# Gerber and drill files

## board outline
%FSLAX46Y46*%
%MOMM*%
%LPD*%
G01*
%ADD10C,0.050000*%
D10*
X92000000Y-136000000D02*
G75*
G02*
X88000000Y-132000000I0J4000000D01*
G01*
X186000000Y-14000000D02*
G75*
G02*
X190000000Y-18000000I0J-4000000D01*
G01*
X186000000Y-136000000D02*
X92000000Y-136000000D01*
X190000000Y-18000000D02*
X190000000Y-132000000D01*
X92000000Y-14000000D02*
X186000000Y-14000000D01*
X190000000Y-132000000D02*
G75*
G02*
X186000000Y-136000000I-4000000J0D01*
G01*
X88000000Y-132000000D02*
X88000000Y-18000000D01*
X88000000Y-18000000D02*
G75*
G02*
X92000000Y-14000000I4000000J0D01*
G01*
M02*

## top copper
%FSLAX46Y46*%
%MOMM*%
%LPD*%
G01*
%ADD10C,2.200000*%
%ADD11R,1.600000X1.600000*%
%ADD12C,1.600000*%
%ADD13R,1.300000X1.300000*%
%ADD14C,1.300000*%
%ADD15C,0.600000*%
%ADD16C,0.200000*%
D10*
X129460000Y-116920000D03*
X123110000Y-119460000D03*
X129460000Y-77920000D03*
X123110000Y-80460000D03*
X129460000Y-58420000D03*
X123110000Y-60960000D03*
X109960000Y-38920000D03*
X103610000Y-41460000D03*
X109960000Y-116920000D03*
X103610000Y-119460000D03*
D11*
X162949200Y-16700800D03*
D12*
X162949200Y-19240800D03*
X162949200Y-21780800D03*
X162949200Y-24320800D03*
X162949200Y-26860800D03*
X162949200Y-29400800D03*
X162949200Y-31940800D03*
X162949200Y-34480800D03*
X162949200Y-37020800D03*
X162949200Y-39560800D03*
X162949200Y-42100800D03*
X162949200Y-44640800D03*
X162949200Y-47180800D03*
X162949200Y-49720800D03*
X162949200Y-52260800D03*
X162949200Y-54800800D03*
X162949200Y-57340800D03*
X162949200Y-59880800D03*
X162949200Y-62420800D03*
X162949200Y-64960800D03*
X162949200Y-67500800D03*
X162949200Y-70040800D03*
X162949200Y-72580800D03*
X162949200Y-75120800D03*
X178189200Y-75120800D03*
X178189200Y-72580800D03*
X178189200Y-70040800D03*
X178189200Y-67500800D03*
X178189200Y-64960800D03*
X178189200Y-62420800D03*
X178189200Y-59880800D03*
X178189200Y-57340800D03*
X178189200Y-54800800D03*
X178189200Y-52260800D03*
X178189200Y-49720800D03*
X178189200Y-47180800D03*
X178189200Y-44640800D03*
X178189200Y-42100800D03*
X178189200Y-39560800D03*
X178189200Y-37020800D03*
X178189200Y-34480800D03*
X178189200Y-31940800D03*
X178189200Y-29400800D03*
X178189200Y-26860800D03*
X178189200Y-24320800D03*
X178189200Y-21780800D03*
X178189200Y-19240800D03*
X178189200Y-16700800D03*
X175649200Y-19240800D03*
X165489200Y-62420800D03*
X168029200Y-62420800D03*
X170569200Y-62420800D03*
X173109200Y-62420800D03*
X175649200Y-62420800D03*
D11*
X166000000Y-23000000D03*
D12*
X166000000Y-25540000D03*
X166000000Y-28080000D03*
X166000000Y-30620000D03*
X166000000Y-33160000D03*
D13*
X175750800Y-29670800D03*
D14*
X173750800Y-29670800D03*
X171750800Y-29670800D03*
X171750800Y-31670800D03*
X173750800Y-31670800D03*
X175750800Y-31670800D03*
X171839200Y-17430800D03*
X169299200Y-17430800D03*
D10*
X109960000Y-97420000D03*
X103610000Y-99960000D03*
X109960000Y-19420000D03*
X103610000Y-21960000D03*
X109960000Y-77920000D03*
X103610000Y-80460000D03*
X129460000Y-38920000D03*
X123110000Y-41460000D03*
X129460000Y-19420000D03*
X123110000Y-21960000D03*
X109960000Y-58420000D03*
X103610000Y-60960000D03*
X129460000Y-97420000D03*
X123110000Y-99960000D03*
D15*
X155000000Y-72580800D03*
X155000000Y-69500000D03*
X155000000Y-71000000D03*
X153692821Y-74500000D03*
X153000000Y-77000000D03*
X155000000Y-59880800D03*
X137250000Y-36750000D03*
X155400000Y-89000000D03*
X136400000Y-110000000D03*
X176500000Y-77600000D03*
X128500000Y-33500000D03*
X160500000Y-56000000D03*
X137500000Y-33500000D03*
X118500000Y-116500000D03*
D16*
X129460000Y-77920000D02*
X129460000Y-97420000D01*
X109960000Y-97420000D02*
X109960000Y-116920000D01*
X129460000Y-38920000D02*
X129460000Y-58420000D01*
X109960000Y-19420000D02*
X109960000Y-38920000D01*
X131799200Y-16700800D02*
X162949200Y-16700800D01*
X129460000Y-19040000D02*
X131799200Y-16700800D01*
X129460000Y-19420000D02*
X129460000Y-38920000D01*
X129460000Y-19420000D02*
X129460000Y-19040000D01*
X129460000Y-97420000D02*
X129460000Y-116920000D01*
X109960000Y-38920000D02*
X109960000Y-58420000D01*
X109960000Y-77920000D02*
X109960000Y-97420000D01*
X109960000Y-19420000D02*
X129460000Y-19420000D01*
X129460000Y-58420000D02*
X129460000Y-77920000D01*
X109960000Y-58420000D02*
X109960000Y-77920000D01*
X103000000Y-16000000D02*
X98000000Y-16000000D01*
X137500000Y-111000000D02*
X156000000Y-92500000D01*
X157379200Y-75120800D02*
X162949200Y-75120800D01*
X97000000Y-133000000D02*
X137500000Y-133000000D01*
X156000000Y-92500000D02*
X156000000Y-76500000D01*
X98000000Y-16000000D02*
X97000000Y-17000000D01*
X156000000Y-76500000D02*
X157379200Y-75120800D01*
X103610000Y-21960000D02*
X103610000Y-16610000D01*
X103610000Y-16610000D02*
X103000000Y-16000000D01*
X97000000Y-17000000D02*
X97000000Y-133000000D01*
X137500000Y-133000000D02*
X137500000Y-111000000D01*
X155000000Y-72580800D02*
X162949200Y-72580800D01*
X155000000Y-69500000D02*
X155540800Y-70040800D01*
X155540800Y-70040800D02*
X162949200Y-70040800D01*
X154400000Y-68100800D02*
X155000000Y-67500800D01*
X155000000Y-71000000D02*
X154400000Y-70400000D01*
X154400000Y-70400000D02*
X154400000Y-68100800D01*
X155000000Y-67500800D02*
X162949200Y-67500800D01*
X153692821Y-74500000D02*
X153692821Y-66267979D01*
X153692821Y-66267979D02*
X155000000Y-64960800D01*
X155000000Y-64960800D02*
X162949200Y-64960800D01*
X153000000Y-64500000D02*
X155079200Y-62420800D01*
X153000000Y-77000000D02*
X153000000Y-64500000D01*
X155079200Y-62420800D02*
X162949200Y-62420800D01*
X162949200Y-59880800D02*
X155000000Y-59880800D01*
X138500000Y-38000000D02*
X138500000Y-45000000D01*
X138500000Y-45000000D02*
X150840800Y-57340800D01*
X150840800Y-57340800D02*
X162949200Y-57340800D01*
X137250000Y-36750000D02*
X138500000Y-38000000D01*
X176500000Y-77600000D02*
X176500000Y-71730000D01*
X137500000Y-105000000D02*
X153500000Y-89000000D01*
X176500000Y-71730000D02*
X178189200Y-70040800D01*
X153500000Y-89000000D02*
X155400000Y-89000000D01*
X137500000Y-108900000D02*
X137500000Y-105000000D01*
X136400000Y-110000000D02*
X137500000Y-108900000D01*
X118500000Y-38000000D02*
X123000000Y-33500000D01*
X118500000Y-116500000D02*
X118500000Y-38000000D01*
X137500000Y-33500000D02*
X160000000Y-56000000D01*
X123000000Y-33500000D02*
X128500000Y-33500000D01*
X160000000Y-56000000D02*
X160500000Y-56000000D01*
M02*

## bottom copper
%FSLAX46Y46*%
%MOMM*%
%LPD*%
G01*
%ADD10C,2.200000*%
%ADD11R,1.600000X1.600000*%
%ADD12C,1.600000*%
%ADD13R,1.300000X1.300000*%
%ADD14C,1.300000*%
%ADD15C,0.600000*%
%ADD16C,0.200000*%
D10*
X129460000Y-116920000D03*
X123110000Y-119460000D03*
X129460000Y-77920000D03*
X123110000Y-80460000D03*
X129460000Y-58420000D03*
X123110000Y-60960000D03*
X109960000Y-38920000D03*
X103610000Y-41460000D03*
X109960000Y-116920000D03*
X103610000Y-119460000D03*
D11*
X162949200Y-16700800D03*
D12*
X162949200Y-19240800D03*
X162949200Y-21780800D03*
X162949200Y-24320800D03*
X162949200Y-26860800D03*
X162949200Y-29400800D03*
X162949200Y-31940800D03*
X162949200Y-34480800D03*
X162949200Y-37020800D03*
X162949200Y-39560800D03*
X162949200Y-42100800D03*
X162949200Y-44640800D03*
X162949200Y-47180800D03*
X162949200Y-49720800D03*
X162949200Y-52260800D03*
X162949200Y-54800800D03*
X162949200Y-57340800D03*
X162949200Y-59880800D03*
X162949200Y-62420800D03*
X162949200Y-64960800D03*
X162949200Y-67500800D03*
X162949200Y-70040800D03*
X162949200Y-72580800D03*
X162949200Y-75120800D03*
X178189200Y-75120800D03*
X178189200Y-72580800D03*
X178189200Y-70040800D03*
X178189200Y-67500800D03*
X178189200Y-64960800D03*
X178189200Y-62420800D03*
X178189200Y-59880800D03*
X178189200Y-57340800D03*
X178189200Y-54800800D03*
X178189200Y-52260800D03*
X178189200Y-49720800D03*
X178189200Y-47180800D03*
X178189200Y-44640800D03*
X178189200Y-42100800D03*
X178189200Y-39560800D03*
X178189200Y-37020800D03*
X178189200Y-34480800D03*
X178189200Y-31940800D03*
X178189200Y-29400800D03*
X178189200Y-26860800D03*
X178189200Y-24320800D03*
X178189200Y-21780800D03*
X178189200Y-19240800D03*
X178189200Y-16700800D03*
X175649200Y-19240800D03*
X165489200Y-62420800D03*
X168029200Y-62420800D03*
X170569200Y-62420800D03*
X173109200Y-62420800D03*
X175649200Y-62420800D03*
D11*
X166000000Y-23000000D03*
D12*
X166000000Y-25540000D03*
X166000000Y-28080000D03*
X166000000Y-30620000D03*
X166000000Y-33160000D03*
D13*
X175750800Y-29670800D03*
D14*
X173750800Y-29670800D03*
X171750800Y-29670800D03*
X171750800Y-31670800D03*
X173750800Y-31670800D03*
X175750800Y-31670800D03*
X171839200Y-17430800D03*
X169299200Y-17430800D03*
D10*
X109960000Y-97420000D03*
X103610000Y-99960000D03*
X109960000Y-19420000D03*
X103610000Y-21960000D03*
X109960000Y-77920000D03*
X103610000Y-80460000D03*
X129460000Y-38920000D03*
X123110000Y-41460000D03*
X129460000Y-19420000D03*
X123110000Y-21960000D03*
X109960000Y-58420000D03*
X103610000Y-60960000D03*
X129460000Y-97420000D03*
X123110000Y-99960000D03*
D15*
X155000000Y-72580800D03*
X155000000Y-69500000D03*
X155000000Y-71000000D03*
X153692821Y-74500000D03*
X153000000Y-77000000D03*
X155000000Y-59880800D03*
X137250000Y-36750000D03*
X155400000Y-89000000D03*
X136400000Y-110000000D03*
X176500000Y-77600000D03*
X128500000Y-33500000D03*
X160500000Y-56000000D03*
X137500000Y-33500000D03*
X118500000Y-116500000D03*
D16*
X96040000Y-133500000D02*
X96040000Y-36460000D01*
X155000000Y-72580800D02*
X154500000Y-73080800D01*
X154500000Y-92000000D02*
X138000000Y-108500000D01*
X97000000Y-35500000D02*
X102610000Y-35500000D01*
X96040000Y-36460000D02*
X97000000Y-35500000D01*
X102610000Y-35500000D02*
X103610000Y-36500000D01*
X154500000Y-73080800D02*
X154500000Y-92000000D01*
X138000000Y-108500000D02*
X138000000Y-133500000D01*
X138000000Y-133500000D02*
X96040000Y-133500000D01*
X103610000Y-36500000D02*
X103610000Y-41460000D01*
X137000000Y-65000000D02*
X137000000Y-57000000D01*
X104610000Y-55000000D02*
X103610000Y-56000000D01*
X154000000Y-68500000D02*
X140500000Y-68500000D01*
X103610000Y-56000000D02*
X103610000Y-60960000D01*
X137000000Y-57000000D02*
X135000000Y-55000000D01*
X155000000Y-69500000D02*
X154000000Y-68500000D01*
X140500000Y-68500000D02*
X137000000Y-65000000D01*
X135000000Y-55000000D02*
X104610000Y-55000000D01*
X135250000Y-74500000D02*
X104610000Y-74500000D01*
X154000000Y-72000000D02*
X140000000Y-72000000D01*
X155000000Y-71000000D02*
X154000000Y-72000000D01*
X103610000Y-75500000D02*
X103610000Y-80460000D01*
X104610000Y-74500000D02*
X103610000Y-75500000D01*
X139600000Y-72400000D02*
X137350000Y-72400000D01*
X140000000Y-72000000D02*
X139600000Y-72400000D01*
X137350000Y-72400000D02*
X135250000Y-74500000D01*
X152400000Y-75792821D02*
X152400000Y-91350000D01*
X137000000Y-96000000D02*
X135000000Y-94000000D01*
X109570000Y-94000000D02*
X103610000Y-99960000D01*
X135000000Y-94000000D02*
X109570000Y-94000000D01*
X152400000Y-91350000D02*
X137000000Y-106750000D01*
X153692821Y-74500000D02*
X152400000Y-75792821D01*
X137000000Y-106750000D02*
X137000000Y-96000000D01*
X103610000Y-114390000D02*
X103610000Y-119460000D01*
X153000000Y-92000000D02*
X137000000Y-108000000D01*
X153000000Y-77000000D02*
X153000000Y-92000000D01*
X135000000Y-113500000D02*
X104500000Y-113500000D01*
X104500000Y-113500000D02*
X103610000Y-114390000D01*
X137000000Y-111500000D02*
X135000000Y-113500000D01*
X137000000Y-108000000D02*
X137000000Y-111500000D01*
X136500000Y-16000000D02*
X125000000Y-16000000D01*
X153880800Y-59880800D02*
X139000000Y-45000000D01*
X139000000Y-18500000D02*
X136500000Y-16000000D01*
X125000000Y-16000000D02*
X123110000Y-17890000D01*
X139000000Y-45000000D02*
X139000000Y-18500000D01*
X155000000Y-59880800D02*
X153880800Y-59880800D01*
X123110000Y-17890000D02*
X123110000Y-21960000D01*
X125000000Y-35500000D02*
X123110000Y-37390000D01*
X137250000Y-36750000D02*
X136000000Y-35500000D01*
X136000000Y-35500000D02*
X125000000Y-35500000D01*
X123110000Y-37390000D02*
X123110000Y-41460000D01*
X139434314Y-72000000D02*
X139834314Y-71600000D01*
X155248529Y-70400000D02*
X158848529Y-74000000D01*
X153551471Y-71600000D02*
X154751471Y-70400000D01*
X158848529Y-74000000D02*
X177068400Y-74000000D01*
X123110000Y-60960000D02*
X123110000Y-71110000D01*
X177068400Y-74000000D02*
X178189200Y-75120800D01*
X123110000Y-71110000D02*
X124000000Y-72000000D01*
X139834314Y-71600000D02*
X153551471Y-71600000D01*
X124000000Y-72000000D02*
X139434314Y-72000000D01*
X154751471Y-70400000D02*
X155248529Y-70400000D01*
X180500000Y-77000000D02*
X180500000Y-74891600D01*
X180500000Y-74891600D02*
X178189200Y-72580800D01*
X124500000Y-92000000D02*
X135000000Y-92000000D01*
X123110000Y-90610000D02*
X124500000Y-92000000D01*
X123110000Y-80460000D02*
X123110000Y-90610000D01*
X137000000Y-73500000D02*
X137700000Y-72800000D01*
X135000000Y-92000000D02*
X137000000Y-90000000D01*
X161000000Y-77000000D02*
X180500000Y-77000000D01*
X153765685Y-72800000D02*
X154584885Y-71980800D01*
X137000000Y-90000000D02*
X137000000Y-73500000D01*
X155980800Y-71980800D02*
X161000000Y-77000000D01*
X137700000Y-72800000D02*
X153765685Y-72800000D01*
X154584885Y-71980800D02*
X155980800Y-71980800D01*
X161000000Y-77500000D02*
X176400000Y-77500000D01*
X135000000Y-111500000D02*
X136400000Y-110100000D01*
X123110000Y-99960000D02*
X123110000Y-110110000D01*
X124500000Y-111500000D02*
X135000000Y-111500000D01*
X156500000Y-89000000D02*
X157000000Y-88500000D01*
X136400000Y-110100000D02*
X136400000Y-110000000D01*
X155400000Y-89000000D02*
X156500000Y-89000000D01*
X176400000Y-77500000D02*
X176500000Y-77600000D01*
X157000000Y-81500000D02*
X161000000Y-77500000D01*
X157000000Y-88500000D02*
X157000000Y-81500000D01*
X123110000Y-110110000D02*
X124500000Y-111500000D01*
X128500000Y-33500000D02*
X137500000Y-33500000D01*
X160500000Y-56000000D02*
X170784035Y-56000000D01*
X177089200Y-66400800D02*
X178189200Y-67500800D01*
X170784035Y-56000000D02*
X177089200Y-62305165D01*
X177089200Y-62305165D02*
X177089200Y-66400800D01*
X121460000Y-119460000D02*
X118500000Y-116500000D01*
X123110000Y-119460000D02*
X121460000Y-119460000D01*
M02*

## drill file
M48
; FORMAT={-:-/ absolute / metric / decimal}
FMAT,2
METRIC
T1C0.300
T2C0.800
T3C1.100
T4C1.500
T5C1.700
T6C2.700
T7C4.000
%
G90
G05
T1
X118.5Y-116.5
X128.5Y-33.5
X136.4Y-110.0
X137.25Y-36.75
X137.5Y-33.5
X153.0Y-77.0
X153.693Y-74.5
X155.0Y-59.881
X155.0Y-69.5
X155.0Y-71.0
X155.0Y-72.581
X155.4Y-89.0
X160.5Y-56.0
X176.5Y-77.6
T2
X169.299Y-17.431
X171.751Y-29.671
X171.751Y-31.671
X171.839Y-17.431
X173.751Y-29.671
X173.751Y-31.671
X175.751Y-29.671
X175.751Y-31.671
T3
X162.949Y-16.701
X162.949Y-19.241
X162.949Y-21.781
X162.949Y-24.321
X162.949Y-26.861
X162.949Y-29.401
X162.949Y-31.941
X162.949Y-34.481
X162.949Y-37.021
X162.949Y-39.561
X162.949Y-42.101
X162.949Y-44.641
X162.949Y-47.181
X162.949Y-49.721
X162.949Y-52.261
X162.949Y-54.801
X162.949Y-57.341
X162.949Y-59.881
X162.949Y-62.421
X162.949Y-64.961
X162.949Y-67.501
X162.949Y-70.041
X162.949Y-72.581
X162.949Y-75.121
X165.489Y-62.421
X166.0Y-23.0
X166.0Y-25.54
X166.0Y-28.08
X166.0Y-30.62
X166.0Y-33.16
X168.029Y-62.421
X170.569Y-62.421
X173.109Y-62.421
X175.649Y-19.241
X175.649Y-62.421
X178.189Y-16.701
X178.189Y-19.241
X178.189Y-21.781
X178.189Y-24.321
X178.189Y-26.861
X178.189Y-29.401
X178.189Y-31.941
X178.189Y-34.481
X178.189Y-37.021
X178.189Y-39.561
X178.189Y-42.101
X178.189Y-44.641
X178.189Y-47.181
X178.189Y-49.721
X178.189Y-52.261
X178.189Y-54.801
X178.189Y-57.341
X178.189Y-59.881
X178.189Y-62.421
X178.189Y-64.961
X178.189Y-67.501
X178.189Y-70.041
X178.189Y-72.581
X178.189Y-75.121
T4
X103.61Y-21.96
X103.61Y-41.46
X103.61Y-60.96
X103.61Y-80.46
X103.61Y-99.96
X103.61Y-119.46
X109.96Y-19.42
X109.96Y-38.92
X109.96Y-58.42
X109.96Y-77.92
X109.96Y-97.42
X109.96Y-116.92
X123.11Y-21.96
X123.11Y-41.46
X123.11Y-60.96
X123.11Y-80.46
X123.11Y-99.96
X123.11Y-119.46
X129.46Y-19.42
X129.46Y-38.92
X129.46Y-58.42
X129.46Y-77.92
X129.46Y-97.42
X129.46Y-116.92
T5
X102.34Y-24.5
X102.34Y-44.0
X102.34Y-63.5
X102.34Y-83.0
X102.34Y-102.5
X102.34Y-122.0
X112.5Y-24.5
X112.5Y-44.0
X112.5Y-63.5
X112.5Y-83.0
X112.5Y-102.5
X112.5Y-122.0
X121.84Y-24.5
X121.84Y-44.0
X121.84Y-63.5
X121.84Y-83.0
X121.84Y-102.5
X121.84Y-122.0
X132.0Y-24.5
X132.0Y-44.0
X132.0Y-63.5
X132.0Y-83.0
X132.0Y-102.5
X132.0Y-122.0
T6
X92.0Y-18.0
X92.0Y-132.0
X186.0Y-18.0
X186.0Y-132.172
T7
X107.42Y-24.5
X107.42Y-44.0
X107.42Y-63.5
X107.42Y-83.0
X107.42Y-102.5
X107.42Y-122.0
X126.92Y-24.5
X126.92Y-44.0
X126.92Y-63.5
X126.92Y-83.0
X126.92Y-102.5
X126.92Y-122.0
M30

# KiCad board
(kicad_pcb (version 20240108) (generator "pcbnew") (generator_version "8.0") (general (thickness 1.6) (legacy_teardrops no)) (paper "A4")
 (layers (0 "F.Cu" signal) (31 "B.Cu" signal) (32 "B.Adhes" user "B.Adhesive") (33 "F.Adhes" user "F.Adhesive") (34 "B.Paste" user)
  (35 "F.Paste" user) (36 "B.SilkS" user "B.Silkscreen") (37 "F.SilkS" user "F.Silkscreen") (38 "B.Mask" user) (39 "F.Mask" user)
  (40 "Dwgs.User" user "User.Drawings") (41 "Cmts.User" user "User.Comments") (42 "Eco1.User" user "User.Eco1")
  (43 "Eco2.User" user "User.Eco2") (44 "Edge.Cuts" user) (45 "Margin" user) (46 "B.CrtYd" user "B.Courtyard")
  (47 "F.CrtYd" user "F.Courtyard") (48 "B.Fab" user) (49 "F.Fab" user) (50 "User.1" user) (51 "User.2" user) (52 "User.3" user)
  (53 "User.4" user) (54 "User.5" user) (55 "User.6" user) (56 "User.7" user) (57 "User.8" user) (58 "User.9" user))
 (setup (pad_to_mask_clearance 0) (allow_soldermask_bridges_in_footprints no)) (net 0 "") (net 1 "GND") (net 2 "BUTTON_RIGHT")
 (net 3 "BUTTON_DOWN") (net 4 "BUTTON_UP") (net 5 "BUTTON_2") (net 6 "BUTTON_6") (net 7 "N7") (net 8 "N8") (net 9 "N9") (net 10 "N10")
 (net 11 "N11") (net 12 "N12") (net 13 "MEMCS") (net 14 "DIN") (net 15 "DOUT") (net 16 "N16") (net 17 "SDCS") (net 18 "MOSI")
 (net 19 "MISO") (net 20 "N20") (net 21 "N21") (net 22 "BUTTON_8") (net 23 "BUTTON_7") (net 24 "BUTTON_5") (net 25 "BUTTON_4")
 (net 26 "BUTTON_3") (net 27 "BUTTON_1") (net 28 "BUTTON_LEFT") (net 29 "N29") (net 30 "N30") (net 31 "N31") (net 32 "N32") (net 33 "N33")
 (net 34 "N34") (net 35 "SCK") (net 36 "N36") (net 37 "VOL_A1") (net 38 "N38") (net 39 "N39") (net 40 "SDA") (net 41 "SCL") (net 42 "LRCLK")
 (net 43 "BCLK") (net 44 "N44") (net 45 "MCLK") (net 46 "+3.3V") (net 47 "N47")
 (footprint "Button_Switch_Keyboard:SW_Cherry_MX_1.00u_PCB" (layer "F.Cu") (at 129.46 116.92)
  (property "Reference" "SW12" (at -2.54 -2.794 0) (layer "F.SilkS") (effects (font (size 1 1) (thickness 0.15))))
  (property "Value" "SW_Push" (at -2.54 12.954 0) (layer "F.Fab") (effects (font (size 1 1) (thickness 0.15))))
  (pad "" np_thru_hole circle (at -7.62 5.08) (size 1.7 1.7) (drill 1.7) (layers "*.Cu" "*.Mask"))
  (pad "" np_thru_hole circle (at -2.54 5.08) (size 4 4) (drill 4) (layers "*.Cu" "*.Mask"))
  (pad "" np_thru_hole circle (at 2.54 5.08) (size 1.7 1.7) (drill 1.7) (layers "*.Cu" "*.Mask"))
  (pad "1" thru_hole circle (at 0 0) (size 2.2 2.2) (drill 1.5) (layers "*.Cu" "*.Mask") (remove_unused_layers no) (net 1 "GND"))
  (pad "2" thru_hole circle (at -6.35 2.54) (size 2.2 2.2) (drill 1.5) (layers "*.Cu" "*.Mask") (remove_unused_layers no)
   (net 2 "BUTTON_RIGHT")))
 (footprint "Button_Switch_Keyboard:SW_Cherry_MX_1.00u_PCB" (layer "F.Cu") (at 129.46 77.92)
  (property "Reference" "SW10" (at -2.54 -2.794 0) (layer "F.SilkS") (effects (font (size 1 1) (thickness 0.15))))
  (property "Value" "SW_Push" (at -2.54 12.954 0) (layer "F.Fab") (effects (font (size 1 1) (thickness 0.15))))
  (pad "" np_thru_hole circle (at -7.62 5.08) (size 1.7 1.7) (drill 1.7) (layers "*.Cu" "*.Mask"))
  (pad "" np_thru_hole circle (at -2.54 5.08) (size 4 4) (drill 4) (layers "*.Cu" "*.Mask"))
  (pad "" np_thru_hole circle (at 2.54 5.08) (size 1.7 1.7) (drill 1.7) (layers "*.Cu" "*.Mask"))
  (pad "1" thru_hole circle (at 0 0) (size 2.2 2.2) (drill 1.5) (layers "*.Cu" "*.Mask") (remove_unused_layers no) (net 1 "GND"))
  (pad "2" thru_hole circle (at -6.35 2.54) (size 2.2 2.2) (drill 1.5) (layers "*.Cu" "*.Mask") (remove_unused_layers no)
   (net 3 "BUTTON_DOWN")))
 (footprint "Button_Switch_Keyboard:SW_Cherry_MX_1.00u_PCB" (layer "F.Cu") (at 129.46 58.42)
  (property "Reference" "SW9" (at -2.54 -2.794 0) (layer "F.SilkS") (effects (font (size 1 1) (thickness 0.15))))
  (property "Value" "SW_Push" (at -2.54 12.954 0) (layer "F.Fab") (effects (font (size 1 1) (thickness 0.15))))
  (pad "" np_thru_hole circle (at -7.62 5.08) (size 1.7 1.7) (drill 1.7) (layers "*.Cu" "*.Mask"))
  (pad "" np_thru_hole circle (at -2.54 5.08) (size 4 4) (drill 4) (layers "*.Cu" "*.Mask"))
  (pad "" np_thru_hole circle (at 2.54 5.08) (size 1.7 1.7) (drill 1.7) (layers "*.Cu" "*.Mask"))
  (pad "1" thru_hole circle (at 0 0) (size 2.2 2.2) (drill 1.5) (layers "*.Cu" "*.Mask") (remove_unused_layers no) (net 1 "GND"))
  (pad "2" thru_hole circle (at -6.35 2.54) (size 2.2 2.2) (drill 1.5) (layers "*.Cu" "*.Mask") (remove_unused_layers no)
   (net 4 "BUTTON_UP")))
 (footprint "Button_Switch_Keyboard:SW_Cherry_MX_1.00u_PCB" (layer "F.Cu") (at 109.96 38.92)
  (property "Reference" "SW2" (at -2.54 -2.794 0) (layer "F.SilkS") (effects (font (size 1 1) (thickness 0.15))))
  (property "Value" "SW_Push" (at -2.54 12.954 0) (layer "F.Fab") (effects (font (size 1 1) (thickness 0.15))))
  (pad "" np_thru_hole circle (at -7.62 5.08) (size 1.7 1.7) (drill 1.7) (layers "*.Cu" "*.Mask"))
  (pad "" np_thru_hole circle (at -2.54 5.08) (size 4 4) (drill 4) (layers "*.Cu" "*.Mask"))
  (pad "" np_thru_hole circle (at 2.54 5.08) (size 1.7 1.7) (drill 1.7) (layers "*.Cu" "*.Mask"))
  (pad "1" thru_hole circle (at 0 0) (size 2.2 2.2) (drill 1.5) (layers "*.Cu" "*.Mask") (remove_unused_layers no) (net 1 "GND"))
  (pad "2" thru_hole circle (at -6.35 2.54) (size 2.2 2.2) (drill 1.5) (layers "*.Cu" "*.Mask") (remove_unused_layers no) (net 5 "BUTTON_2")))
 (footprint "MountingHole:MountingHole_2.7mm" (layer "F.Cu") (at 92 18)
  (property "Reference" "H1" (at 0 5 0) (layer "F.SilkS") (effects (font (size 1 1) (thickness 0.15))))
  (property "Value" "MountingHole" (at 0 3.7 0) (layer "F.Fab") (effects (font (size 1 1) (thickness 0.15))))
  (pad "" np_thru_hole circle (at 0 0) (size 2.7 2.7) (drill 2.7) (layers "*.Cu" "*.Mask")))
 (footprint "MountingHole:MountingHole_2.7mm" (layer "F.Cu") (at 186 18)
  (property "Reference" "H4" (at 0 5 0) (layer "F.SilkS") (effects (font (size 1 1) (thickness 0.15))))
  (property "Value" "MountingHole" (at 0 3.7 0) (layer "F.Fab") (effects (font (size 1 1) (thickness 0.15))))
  (pad "" np_thru_hole circle (at 0 0) (size 2.7 2.7) (drill 2.7) (layers "*.Cu" "*.Mask")))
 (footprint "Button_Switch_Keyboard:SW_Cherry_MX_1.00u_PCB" (layer "F.Cu") (at 109.96 116.92)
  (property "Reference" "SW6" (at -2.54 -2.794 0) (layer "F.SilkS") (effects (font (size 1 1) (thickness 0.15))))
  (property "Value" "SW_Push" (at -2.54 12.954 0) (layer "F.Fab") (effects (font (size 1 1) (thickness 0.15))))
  (pad "" np_thru_hole circle (at -7.62 5.08) (size 1.7 1.7) (drill 1.7) (layers "*.Cu" "*.Mask"))
  (pad "" np_thru_hole circle (at -2.54 5.08) (size 4 4) (drill 4) (layers "*.Cu" "*.Mask"))
  (pad "" np_thru_hole circle (at 2.54 5.08) (size 1.7 1.7) (drill 1.7) (layers "*.Cu" "*.Mask"))
  (pad "1" thru_hole circle (at 0 0) (size 2.2 2.2) (drill 1.5) (layers "*.Cu" "*.Mask") (remove_unused_layers no) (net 1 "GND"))
  (pad "2" thru_hole circle (at -6.35 2.54) (size 2.2 2.2) (drill 1.5) (layers "*.Cu" "*.Mask") (remove_unused_layers no) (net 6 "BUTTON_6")))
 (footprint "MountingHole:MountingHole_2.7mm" (layer "F.Cu") (at 186 132.171573)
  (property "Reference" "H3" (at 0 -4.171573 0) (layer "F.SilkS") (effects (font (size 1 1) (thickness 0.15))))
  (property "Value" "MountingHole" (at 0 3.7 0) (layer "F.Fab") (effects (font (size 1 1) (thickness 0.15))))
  (pad "" np_thru_hole circle (at 0 0) (size 2.7 2.7) (drill 2.7) (layers "*.Cu" "*.Mask")))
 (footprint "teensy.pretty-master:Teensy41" (layer "F.Cu") (at 170.5692 45.9108 -90)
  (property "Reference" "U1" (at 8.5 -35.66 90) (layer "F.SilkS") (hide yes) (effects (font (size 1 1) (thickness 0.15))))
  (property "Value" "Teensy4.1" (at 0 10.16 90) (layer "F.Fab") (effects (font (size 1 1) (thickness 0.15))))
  (pad "1" thru_hole rect (at -29.21 7.62 270) (size 1.6 1.6) (drill 1.1) (layers "*.Cu" "*.Mask") (remove_unused_layers no) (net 1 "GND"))
  (pad "2" thru_hole circle (at -26.67 7.62 270) (size 1.6 1.6) (drill 1.1) (layers "*.Cu" "*.Mask") (remove_unused_layers no) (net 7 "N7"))
  (pad "3" thru_hole circle (at -24.13 7.62 270) (size 1.6 1.6) (drill 1.1) (layers "*.Cu" "*.Mask") (remove_unused_layers no) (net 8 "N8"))
  (pad "4" thru_hole circle (at -21.59 7.62 270) (size 1.6 1.6) (drill 1.1) (layers "*.Cu" "*.Mask") (remove_unused_layers no) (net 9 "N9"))
  (pad "5" thru_hole circle (at -19.05 7.62 270) (size 1.6 1.6) (drill 1.1) (layers "*.Cu" "*.Mask") (remove_unused_layers no)
   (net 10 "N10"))
  (pad "6" thru_hole circle (at -16.51 7.62 270) (size 1.6 1.6) (drill 1.1) (layers "*.Cu" "*.Mask") (remove_unused_layers no)
   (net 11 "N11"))
  (pad "7" thru_hole circle (at -13.97 7.62 270) (size 1.6 1.6) (drill 1.1) (layers "*.Cu" "*.Mask") (remove_unused_layers no)
   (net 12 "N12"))
  (pad "8" thru_hole circle (at -11.43 7.62 270) (size 1.6 1.6) (drill 1.1) (layers "*.Cu" "*.Mask") (remove_unused_layers no)
   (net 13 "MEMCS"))
  (pad "9" thru_hole circle (at -8.89 7.62 270) (size 1.6 1.6) (drill 1.1) (layers "*.Cu" "*.Mask") (remove_unused_layers no) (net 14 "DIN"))
  (pad "10" thru_hole circle (at -6.35 7.62 270) (size 1.6 1.6) (drill 1.1) (layers "*.Cu" "*.Mask") (remove_unused_layers no)
   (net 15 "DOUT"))
  (pad "11" thru_hole circle (at -3.81 7.62 270) (size 1.6 1.6) (drill 1.1) (layers "*.Cu" "*.Mask") (remove_unused_layers no)
   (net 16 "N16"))
  (pad "12" thru_hole circle (at -1.27 7.62 270) (size 1.6 1.6) (drill 1.1) (layers "*.Cu" "*.Mask") (remove_unused_layers no)
   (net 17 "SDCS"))
  (pad "13" thru_hole circle (at 1.27 7.62 270) (size 1.6 1.6) (drill 1.1) (layers "*.Cu" "*.Mask") (remove_unused_layers no)
   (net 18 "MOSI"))
  (pad "14" thru_hole circle (at 3.81 7.62 270) (size 1.6 1.6) (drill 1.1) (layers "*.Cu" "*.Mask") (remove_unused_layers no)
   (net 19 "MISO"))
  (pad "15" thru_hole circle (at 6.35 7.62 270) (size 1.6 1.6) (drill 1.1) (layers "*.Cu" "*.Mask") (remove_unused_layers no) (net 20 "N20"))
  (pad "16" thru_hole circle (at 8.89 7.62 270) (size 1.6 1.6) (drill 1.1) (layers "*.Cu" "*.Mask") (remove_unused_layers no) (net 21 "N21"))
  (pad "17" thru_hole circle (at 11.43 7.62 270) (size 1.6 1.6) (drill 1.1) (layers "*.Cu" "*.Mask") (remove_unused_layers no)
   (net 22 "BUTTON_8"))
  (pad "18" thru_hole circle (at 13.97 7.62 270) (size 1.6 1.6) (drill 1.1) (layers "*.Cu" "*.Mask") (remove_unused_layers no)
   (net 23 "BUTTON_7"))
  (pad "19" thru_hole circle (at 16.51 7.62 270) (size 1.6 1.6) (drill 1.1) (layers "*.Cu" "*.Mask") (remove_unused_layers no)
   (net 6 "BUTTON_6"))
  (pad "20" thru_hole circle (at 19.05 7.62 270) (size 1.6 1.6) (drill 1.1) (layers "*.Cu" "*.Mask") (remove_unused_layers no)
   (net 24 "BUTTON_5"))
  (pad "21" thru_hole circle (at 21.59 7.62 270) (size 1.6 1.6) (drill 1.1) (layers "*.Cu" "*.Mask") (remove_unused_layers no)
   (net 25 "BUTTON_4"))
  (pad "22" thru_hole circle (at 24.13 7.62 270) (size 1.6 1.6) (drill 1.1) (layers "*.Cu" "*.Mask") (remove_unused_layers no)
   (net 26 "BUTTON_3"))
  (pad "23" thru_hole circle (at 26.67 7.62 270) (size 1.6 1.6) (drill 1.1) (layers "*.Cu" "*.Mask") (remove_unused_layers no)
   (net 5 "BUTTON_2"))
  (pad "24" thru_hole circle (at 29.21 7.62 270) (size 1.6 1.6) (drill 1.1) (layers "*.Cu" "*.Mask") (remove_unused_layers no)
   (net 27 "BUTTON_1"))
  (pad "25" thru_hole circle (at 29.21 -7.62 270) (size 1.6 1.6) (drill 1.1) (layers "*.Cu" "*.Mask") (remove_unused_layers no)
   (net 4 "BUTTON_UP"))
  (pad "26" thru_hole circle (at 26.67 -7.62 270) (size 1.6 1.6) (drill 1.1) (layers "*.Cu" "*.Mask") (remove_unused_layers no)
   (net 3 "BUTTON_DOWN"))
  (pad "27" thru_hole circle (at 24.13 -7.62 270) (size 1.6 1.6) (drill 1.1) (layers "*.Cu" "*.Mask") (remove_unused_layers no)
   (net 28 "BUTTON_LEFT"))
  (pad "28" thru_hole circle (at 21.59 -7.62 270) (size 1.6 1.6) (drill 1.1) (layers "*.Cu" "*.Mask") (remove_unused_layers no)
   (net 2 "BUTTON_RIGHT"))
  (pad "29" thru_hole circle (at 19.05 -7.62 270) (size 1.6 1.6) (drill 1.1) (layers "*.Cu" "*.Mask") (remove_unused_layers no)
   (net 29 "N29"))
  (pad "30" thru_hole circle (at 16.51 -7.62 270) (size 1.6 1.6) (drill 1.1) (layers "*.Cu" "*.Mask") (remove_unused_layers no)
   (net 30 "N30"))
  (pad "31" thru_hole circle (at 13.97 -7.62 270) (size 1.6 1.6) (drill 1.1) (layers "*.Cu" "*.Mask") (remove_unused_layers no)
   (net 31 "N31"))
  (pad "32" thru_hole circle (at 11.43 -7.62 270) (size 1.6 1.6) (drill 1.1) (layers "*.Cu" "*.Mask") (remove_unused_layers no)
   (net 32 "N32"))
  (pad "33" thru_hole circle (at 8.89 -7.62 270) (size 1.6 1.6) (drill 1.1) (layers "*.Cu" "*.Mask") (remove_unused_layers no)
   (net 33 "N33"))
  (pad "34" thru_hole circle (at 6.35 -7.62 270) (size 1.6 1.6) (drill 1.1) (layers "*.Cu" "*.Mask") (remove_unused_layers no)
   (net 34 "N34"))
  (pad "35" thru_hole circle (at 3.81 -7.62 270) (size 1.6 1.6) (drill 1.1) (layers "*.Cu" "*.Mask") (remove_unused_layers no)
   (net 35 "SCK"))
  (pad "36" thru_hole circle (at 1.27 -7.62 270) (size 1.6 1.6) (drill 1.1) (layers "*.Cu" "*.Mask") (remove_unused_layers no)
   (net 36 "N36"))
  (pad "37" thru_hole circle (at -1.27 -7.62 270) (size 1.6 1.6) (drill 1.1) (layers "*.Cu" "*.Mask") (remove_unused_layers no)
   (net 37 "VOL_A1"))
  (pad "38" thru_hole circle (at -3.81 -7.62 270) (size 1.6 1.6) (drill 1.1) (layers "*.Cu" "*.Mask") (remove_unused_layers no)
   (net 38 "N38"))
  (pad "39" thru_hole circle (at -6.35 -7.62 270) (size 1.6 1.6) (drill 1.1) (layers "*.Cu" "*.Mask") (remove_unused_layers no)
   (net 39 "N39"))
  (pad "40" thru_hole circle (at -8.89 -7.62 270) (size 1.6 1.6) (drill 1.1) (layers "*.Cu" "*.Mask") (remove_unused_layers no)
   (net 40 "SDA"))
  (pad "41" thru_hole circle (at -11.43 -7.62 270) (size 1.6 1.6) (drill 1.1) (layers "*.Cu" "*.Mask") (remove_unused_layers no)
   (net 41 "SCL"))
  (pad "42" thru_hole circle (at -13.97 -7.62 270) (size 1.6 1.6) (drill 1.1) (layers "*.Cu" "*.Mask") (remove_unused_layers no)
   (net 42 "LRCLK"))
  (pad "43" thru_hole circle (at -16.51 -7.62 270) (size 1.6 1.6) (drill 1.1) (layers "*.Cu" "*.Mask") (remove_unused_layers no)
   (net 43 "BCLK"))
  (pad "44" thru_hole circle (at -19.05 -7.62 270) (size 1.6 1.6) (drill 1.1) (layers "*.Cu" "*.Mask") (remove_unused_layers no)
   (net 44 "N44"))
  (pad "45" thru_hole circle (at -21.59 -7.62 270) (size 1.6 1.6) (drill 1.1) (layers "*.Cu" "*.Mask") (remove_unused_layers no)
   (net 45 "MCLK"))
  (pad "46" thru_hole circle (at -24.13 -7.62 270) (size 1.6 1.6) (drill 1.1) (layers "*.Cu" "*.Mask") (remove_unused_layers no)
   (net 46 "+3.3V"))
  (pad "47" thru_hole circle (at -26.67 -7.62 270) (size 1.6 1.6) (drill 1.1) (layers "*.Cu" "*.Mask") (remove_unused_layers no)
   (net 1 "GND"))
  (pad "48" thru_hole circle (at -29.21 -7.62 270) (size 1.6 1.6) (drill 1.1) (layers "*.Cu" "*.Mask") (remove_unused_layers no)
   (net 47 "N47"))
  (pad "49" thru_hole circle (at -26.67 -5.08 270) (size 1.6 1.6) (drill 1.1) (layers "*.Cu" "*.Mask") (remove_unused_layers no))
  (pad "50" thru_hole circle (at 16.51 5.08 270) (size 1.6 1.6) (drill 1.1) (layers "*.Cu" "*.Mask") (remove_unused_layers no))
  (pad "51" thru_hole circle (at 16.51 2.54 270) (size 1.6 1.6) (drill 1.1) (layers "*.Cu" "*.Mask") (remove_unused_layers no))
  (pad "52" thru_hole circle (at 16.51 0 270) (size 1.6 1.6) (drill 1.1) (layers "*.Cu" "*.Mask") (remove_unused_layers no))
  (pad "53" thru_hole circle (at 16.51 -2.54 270) (size 1.6 1.6) (drill 1.1) (layers "*.Cu" "*.Mask") (remove_unused_layers no))
  (pad "54" thru_hole circle (at 16.51 -5.08 270) (size 1.6 1.6) (drill 1.1) (layers "*.Cu" "*.Mask") (remove_unused_layers no))
  (pad "55" thru_hole rect (at -22.9108 4.5692 270) (size 1.6 1.6) (drill 1.1) (layers "*.Cu" "*.Mask") (remove_unused_layers no))
  (pad "56" thru_hole circle (at -20.3708 4.5692 270) (size 1.6 1.6) (drill 1.1) (layers "*.Cu" "*.Mask") (remove_unused_layers no))
  (pad "57" thru_hole circle (at -17.8308 4.5692 270) (size 1.6 1.6) (drill 1.1) (layers "*.Cu" "*.Mask") (remove_unused_layers no))
  (pad "58" thru_hole circle (at -15.2908 4.5692 270) (size 1.6 1.6) (drill 1.1) (layers "*.Cu" "*.Mask") (remove_unused_layers no))
  (pad "59" thru_hole circle (at -12.7508 4.5692 270) (size 1.6 1.6) (drill 1.1) (layers "*.Cu" "*.Mask") (remove_unused_layers no))
  (pad "60" thru_hole rect (at -16.24 -5.1816 270) (size 1.3 1.3) (drill 0.8) (layers "*.Cu" "*.Mask") (remove_unused_layers no))
  (pad "61" thru_hole circle (at -16.24 -3.1816 270) (size 1.3 1.3) (drill 0.8) (layers "*.Cu" "*.Mask") (remove_unused_layers no))
  (pad "62" thru_hole circle (at -16.24 -1.1816 270) (size 1.3 1.3) (drill 0.8) (layers "*.Cu" "*.Mask") (remove_unused_layers no))
  (pad "63" thru_hole circle (at -14.24 -1.1816 270) (size 1.3 1.3) (drill 0.8) (layers "*.Cu" "*.Mask") (remove_unused_layers no))
  (pad "64" thru_hole circle (at -14.24 -3.1816 270) (size 1.3 1.3) (drill 0.8) (layers "*.Cu" "*.Mask") (remove_unused_layers no))
  (pad "65" thru_hole circle (at -14.24 -5.1816 270) (size 1.3 1.3) (drill 0.8) (layers "*.Cu" "*.Mask") (remove_unused_layers no))
  (pad "66" thru_hole circle (at -28.48 -1.27 270) (size 1.3 1.3) (drill 0.8) (layers "*.Cu" "*.Mask") (remove_unused_layers no))
  (pad "67" thru_hole circle (at -28.48 1.27 270) (size 1.3 1.3) (drill 0.8) (layers "*.Cu" "*.Mask") (remove_unused_layers no)))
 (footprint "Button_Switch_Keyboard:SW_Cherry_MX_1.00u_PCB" (layer "F.Cu") (at 109.96 97.42)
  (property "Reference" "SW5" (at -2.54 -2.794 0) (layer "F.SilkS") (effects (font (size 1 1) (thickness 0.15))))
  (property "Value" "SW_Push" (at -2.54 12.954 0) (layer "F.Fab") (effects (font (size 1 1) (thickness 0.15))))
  (pad "" np_thru_hole circle (at -7.62 5.08) (size 1.7 1.7) (drill 1.7) (layers "*.Cu" "*.Mask"))
  (pad "" np_thru_hole circle (at -2.54 5.08) (size 4 4) (drill 4) (layers "*.Cu" "*.Mask"))
  (pad "" np_thru_hole circle (at 2.54 5.08) (size 1.7 1.7) (drill 1.7) (layers "*.Cu" "*.Mask"))
  (pad "1" thru_hole circle (at 0 0) (size 2.2 2.2) (drill 1.5) (layers "*.Cu" "*.Mask") (remove_unused_layers no) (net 1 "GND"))
  (pad "2" thru_hole circle (at -6.35 2.54) (size 2.2 2.2) (drill 1.5) (layers "*.Cu" "*.Mask") (remove_unused_layers no)
   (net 24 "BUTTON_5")))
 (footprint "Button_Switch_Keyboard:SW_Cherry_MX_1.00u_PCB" (layer "F.Cu") (at 109.96 19.42)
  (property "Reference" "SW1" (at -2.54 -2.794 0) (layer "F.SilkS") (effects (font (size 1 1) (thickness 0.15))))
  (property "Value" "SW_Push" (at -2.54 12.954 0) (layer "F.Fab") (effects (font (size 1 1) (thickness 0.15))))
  (pad "" np_thru_hole circle (at -7.62 5.08) (size 1.7 1.7) (drill 1.7) (layers "*.Cu" "*.Mask"))
  (pad "" np_thru_hole circle (at -2.54 5.08) (size 4 4) (drill 4) (layers "*.Cu" "*.Mask"))
  (pad "" np_thru_hole circle (at 2.54 5.08) (size 1.7 1.7) (drill 1.7) (layers "*.Cu" "*.Mask"))
  (pad "1" thru_hole circle (at 0 0) (size 2.2 2.2) (drill 1.5) (layers "*.Cu" "*.Mask") (remove_unused_layers no) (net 1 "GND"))
  (pad "2" thru_hole circle (at -6.35 2.54) (size 2.2 2.2) (drill 1.5) (layers "*.Cu" "*.Mask") (remove_unused_layers no)
   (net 27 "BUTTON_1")))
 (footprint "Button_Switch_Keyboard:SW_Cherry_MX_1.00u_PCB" (layer "F.Cu") (at 109.96 77.92)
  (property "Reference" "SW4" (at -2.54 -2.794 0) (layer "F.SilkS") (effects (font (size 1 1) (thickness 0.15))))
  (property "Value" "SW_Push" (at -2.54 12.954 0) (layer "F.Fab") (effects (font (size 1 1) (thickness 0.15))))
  (pad "" np_thru_hole circle (at -7.62 5.08) (size 1.7 1.7) (drill 1.7) (layers "*.Cu" "*.Mask"))
  (pad "" np_thru_hole circle (at -2.54 5.08) (size 4 4) (drill 4) (layers "*.Cu" "*.Mask"))
  (pad "" np_thru_hole circle (at 2.54 5.08) (size 1.7 1.7) (drill 1.7) (layers "*.Cu" "*.Mask"))
  (pad "1" thru_hole circle (at 0 0) (size 2.2 2.2) (drill 1.5) (layers "*.Cu" "*.Mask") (remove_unused_layers no) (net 1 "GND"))
  (pad "2" thru_hole circle (at -6.35 2.54) (size 2.2 2.2) (drill 1.5) (layers "*.Cu" "*.Mask") (remove_unused_layers no)
   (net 25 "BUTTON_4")))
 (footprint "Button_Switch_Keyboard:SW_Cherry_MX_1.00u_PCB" (layer "F.Cu") (at 129.46 38.92)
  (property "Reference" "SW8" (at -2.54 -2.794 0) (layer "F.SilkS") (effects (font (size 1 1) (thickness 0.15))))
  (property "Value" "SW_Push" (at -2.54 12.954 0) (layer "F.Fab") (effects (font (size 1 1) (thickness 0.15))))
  (pad "" np_thru_hole circle (at -7.62 5.08) (size 1.7 1.7) (drill 1.7) (layers "*.Cu" "*.Mask"))
  (pad "" np_thru_hole circle (at -2.54 5.08) (size 4 4) (drill 4) (layers "*.Cu" "*.Mask"))
  (pad "" np_thru_hole circle (at 2.54 5.08) (size 1.7 1.7) (drill 1.7) (layers "*.Cu" "*.Mask"))
  (pad "1" thru_hole circle (at 0 0) (size 2.2 2.2) (drill 1.5) (layers "*.Cu" "*.Mask") (remove_unused_layers no) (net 1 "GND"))
  (pad "2" thru_hole circle (at -6.35 2.54) (size 2.2 2.2) (drill 1.5) (layers "*.Cu" "*.Mask") (remove_unused_layers no)
   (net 22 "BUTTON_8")))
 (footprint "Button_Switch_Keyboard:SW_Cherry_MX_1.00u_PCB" (layer "F.Cu") (at 129.46 19.42)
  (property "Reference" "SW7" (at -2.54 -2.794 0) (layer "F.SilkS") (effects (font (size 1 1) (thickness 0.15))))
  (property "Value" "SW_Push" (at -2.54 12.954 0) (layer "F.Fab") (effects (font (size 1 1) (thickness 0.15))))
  (pad "" np_thru_hole circle (at -7.62 5.08) (size 1.7 1.7) (drill 1.7) (layers "*.Cu" "*.Mask"))
  (pad "" np_thru_hole circle (at -2.54 5.08) (size 4 4) (drill 4) (layers "*.Cu" "*.Mask"))
  (pad "" np_thru_hole circle (at 2.54 5.08) (size 1.7 1.7) (drill 1.7) (layers "*.Cu" "*.Mask"))
  (pad "1" thru_hole circle (at 0 0) (size 2.2 2.2) (drill 1.5) (layers "*.Cu" "*.Mask") (remove_unused_layers no) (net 1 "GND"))
  (pad "2" thru_hole circle (at -6.35 2.54) (size 2.2 2.2) (drill 1.5) (layers "*.Cu" "*.Mask") (remove_unused_layers no)
   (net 23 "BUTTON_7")))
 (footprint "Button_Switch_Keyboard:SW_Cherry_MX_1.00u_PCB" (layer "F.Cu") (at 109.96 58.42)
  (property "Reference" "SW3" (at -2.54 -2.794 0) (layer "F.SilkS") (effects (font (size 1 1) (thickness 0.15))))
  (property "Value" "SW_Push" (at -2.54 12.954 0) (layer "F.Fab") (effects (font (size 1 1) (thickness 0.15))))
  (pad "" np_thru_hole circle (at -7.62 5.08) (size 1.7 1.7) (drill 1.7) (layers "*.Cu" "*.Mask"))
  (pad "" np_thru_hole circle (at -2.54 5.08) (size 4 4) (drill 4) (layers "*.Cu" "*.Mask"))
  (pad "" np_thru_hole circle (at 2.54 5.08) (size 1.7 1.7) (drill 1.7) (layers "*.Cu" "*.Mask"))
  (pad "1" thru_hole circle (at 0 0) (size 2.2 2.2) (drill 1.5) (layers "*.Cu" "*.Mask") (remove_unused_layers no) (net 1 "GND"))
  (pad "2" thru_hole circle (at -6.35 2.54) (size 2.2 2.2) (drill 1.5) (layers "*.Cu" "*.Mask") (remove_unused_layers no)
   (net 26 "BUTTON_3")))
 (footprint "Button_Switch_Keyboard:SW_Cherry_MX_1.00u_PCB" (layer "F.Cu") (at 129.46 97.42)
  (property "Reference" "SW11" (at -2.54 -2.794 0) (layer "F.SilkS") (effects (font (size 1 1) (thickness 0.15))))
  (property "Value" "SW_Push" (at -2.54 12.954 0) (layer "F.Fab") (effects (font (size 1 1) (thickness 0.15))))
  (pad "" np_thru_hole circle (at -7.62 5.08) (size 1.7 1.7) (drill 1.7) (layers "*.Cu" "*.Mask"))
  (pad "" np_thru_hole circle (at -2.54 5.08) (size 4 4) (drill 4) (layers "*.Cu" "*.Mask"))
  (pad "" np_thru_hole circle (at 2.54 5.08) (size 1.7 1.7) (drill 1.7) (layers "*.Cu" "*.Mask"))
  (pad "1" thru_hole circle (at 0 0) (size 2.2 2.2) (drill 1.5) (layers "*.Cu" "*.Mask") (remove_unused_layers no) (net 1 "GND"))
  (pad "2" thru_hole circle (at -6.35 2.54) (size 2.2 2.2) (drill 1.5) (layers "*.Cu" "*.Mask") (remove_unused_layers no)
   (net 28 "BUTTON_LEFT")))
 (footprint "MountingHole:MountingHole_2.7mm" (layer "F.Cu") (at 92 132)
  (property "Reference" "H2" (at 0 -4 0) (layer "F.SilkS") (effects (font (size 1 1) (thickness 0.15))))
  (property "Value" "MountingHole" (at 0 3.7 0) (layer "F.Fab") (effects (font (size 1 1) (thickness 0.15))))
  (pad "" np_thru_hole circle (at 0 0) (size 2.7 2.7) (drill 2.7) (layers "*.Cu" "*.Mask")))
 (gr_arc (start 92 136) (mid 89.171573 134.828427) (end 88 132) (stroke (width 0.05) (type default)) (layer "Edge.Cuts"))
 (gr_arc (start 186 14) (mid 188.828427 15.171573) (end 190 18) (stroke (width 0.05) (type default)) (layer "Edge.Cuts"))
 (gr_line (start 186 136) (end 92 136) (stroke (width 0.05) (type default)) (layer "Edge.Cuts"))
 (gr_line (start 190 18) (end 190 132) (stroke (width 0.05) (type default)) (layer "Edge.Cuts"))
 (gr_line (start 92 14) (end 186 14) (stroke (width 0.05) (type default)) (layer "Edge.Cuts"))
 (gr_arc (start 190 132) (mid 188.828427 134.828427) (end 186 136) (stroke (width 0.05) (type default)) (layer "Edge.Cuts"))
 (gr_line (start 88 132) (end 88 18) (stroke (width 0.05) (type default)) (layer "Edge.Cuts"))
 (gr_arc (start 88 18) (mid 89.171573 15.171573) (end 92 14) (stroke (width 0.05) (type default)) (layer "Edge.Cuts"))
 (segment (start 129.46 77.92) (end 129.46 97.42) (width 0.2) (layer "F.Cu") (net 1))
 (segment (start 109.96 97.42) (end 109.96 116.92) (width 0.2) (layer "F.Cu") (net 1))
 (segment (start 129.46 38.92) (end 129.46 58.42) (width 0.2) (layer "F.Cu") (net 1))
 (segment (start 109.96 19.42) (end 109.96 38.92) (width 0.2) (layer "F.Cu") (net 1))
 (segment (start 131.7992 16.7008) (end 162.9492 16.7008) (width 0.2) (layer "F.Cu") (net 1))
 (segment (start 129.46 19.04) (end 131.7992 16.7008) (width 0.2) (layer "F.Cu") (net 1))
 (segment (start 129.46 19.42) (end 129.46 38.92) (width 0.2) (layer "F.Cu") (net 1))
 (segment (start 129.46 19.42) (end 129.46 19.04) (width 0.2) (layer "F.Cu") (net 1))
 (segment (start 129.46 97.42) (end 129.46 116.92) (width 0.2) (layer "F.Cu") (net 1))
 (segment (start 109.96 38.92) (end 109.96 58.42) (width 0.2) (layer "F.Cu") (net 1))
 (segment (start 109.96 77.92) (end 109.96 97.42) (width 0.2) (layer "F.Cu") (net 1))
 (segment (start 109.96 19.42) (end 129.46 19.42) (width 0.2) (layer "F.Cu") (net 1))
 (segment (start 129.46 58.42) (end 129.46 77.92) (width 0.2) (layer "F.Cu") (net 1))
 (segment (start 109.96 58.42) (end 109.96 77.92) (width 0.2) (layer "F.Cu") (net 1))
 (segment (start 103 16) (end 98 16) (width 0.2) (layer "F.Cu") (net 27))
 (segment (start 137.5 111) (end 156 92.5) (width 0.2) (layer "F.Cu") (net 27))
 (segment (start 157.3792 75.1208) (end 162.9492 75.1208) (width 0.2) (layer "F.Cu") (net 27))
 (segment (start 97 133) (end 137.5 133) (width 0.2) (layer "F.Cu") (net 27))
 (segment (start 156 92.5) (end 156 76.5) (width 0.2) (layer "F.Cu") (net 27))
 (segment (start 98 16) (end 97 17) (width 0.2) (layer "F.Cu") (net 27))
 (segment (start 156 76.5) (end 157.3792 75.1208) (width 0.2) (layer "F.Cu") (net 27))
 (segment (start 103.61 21.96) (end 103.61 16.61) (width 0.2) (layer "F.Cu") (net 27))
 (segment (start 103.61 16.61) (end 103 16) (width 0.2) (layer "F.Cu") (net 27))
 (segment (start 97 17) (end 97 133) (width 0.2) (layer "F.Cu") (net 27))
 (segment (start 137.5 133) (end 137.5 111) (width 0.2) (layer "F.Cu") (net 27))
 (segment (start 155 72.5808) (end 162.9492 72.5808) (width 0.2) (layer "F.Cu") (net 5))
 (via (at 155 72.5808) (size 0.6) (drill 0.3) (layers "F.Cu" "B.Cu") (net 5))
 (segment (start 96.04 133.5) (end 96.04 36.46) (width 0.2) (layer "B.Cu") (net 5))
 (segment (start 155 72.5808) (end 154.5 73.0808) (width 0.2) (layer "B.Cu") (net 5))
 (segment (start 154.5 92) (end 138 108.5) (width 0.2) (layer "B.Cu") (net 5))
 (segment (start 97 35.5) (end 102.61 35.5) (width 0.2) (layer "B.Cu") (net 5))
 (segment (start 96.04 36.46) (end 97 35.5) (width 0.2) (layer "B.Cu") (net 5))
 (segment (start 102.61 35.5) (end 103.61 36.5) (width 0.2) (layer "B.Cu") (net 5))
 (segment (start 154.5 73.0808) (end 154.5 92) (width 0.2) (layer "B.Cu") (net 5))
 (segment (start 138 108.5) (end 138 133.5) (width 0.2) (layer "B.Cu") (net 5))
 (segment (start 138 133.5) (end 96.04 133.5) (width 0.2) (layer "B.Cu") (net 5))
 (segment (start 103.61 36.5) (end 103.61 41.46) (width 0.2) (layer "B.Cu") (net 5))
 (segment (start 155 69.5) (end 155.5408 70.0408) (width 0.2) (layer "F.Cu") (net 26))
 (segment (start 155.5408 70.0408) (end 162.9492 70.0408) (width 0.2) (layer "F.Cu") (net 26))
 (via (at 155 69.5) (size 0.6) (drill 0.3) (layers "F.Cu" "B.Cu") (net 26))
 (segment (start 137 65) (end 137 57) (width 0.2) (layer "B.Cu") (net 26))
 (segment (start 104.61 55) (end 103.61 56) (width 0.2) (layer "B.Cu") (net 26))
 (segment (start 154 68.5) (end 140.5 68.5) (width 0.2) (layer "B.Cu") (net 26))
 (segment (start 103.61 56) (end 103.61 60.96) (width 0.2) (layer "B.Cu") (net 26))
 (segment (start 137 57) (end 135 55) (width 0.2) (layer "B.Cu") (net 26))
 (segment (start 155 69.5) (end 154 68.5) (width 0.2) (layer "B.Cu") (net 26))
 (segment (start 140.5 68.5) (end 137 65) (width 0.2) (layer "B.Cu") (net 26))
 (segment (start 135 55) (end 104.61 55) (width 0.2) (layer "B.Cu") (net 26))
 (segment (start 154.4 68.1008) (end 155 67.5008) (width 0.2) (layer "F.Cu") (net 25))
 (segment (start 155 71) (end 154.4 70.4) (width 0.2) (layer "F.Cu") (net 25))
 (segment (start 154.4 70.4) (end 154.4 68.1008) (width 0.2) (layer "F.Cu") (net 25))
 (segment (start 155 67.5008) (end 162.9492 67.5008) (width 0.2) (layer "F.Cu") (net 25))
 (via (at 155 71) (size 0.6) (drill 0.3) (layers "F.Cu" "B.Cu") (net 25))
 (segment (start 135.25 74.5) (end 104.61 74.5) (width 0.2) (layer "B.Cu") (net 25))
 (segment (start 154 72) (end 140 72) (width 0.2) (layer "B.Cu") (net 25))
 (segment (start 155 71) (end 154 72) (width 0.2) (layer "B.Cu") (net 25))
 (segment (start 103.61 75.5) (end 103.61 80.46) (width 0.2) (layer "B.Cu") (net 25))
 (segment (start 104.61 74.5) (end 103.61 75.5) (width 0.2) (layer "B.Cu") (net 25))
 (segment (start 139.6 72.4) (end 137.35 72.4) (width 0.2) (layer "B.Cu") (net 25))
 (segment (start 140 72) (end 139.6 72.4) (width 0.2) (layer "B.Cu") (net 25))
 (segment (start 137.35 72.4) (end 135.25 74.5) (width 0.2) (layer "B.Cu") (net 25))
 (segment (start 153.692821 74.5) (end 153.692821 66.267979) (width 0.2) (layer "F.Cu") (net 24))
 (segment (start 153.692821 66.267979) (end 155 64.9608) (width 0.2) (layer "F.Cu") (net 24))
 (segment (start 155 64.9608) (end 162.9492 64.9608) (width 0.2) (layer "F.Cu") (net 24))
 (via (at 153.692821 74.5) (size 0.6) (drill 0.3) (layers "F.Cu" "B.Cu") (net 24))
 (segment (start 152.4 75.792821) (end 152.4 91.35) (width 0.2) (layer "B.Cu") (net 24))
 (segment (start 137 96) (end 135 94) (width 0.2) (layer "B.Cu") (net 24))
 (segment (start 109.57 94) (end 103.61 99.96) (width 0.2) (layer "B.Cu") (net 24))
 (segment (start 135 94) (end 109.57 94) (width 0.2) (layer "B.Cu") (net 24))
 (segment (start 152.4 91.35) (end 137 106.75) (width 0.2) (layer "B.Cu") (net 24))
 (segment (start 153.692821 74.5) (end 152.4 75.792821) (width 0.2) (layer "B.Cu") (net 24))
 (segment (start 137 106.75) (end 137 96) (width 0.2) (layer "B.Cu") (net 24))
 (segment (start 153 64.5) (end 155.0792 62.4208) (width 0.2) (layer "F.Cu") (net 6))
 (segment (start 153 77) (end 153 64.5) (width 0.2) (layer "F.Cu") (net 6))
 (segment (start 155.0792 62.4208) (end 162.9492 62.4208) (width 0.2) (layer "F.Cu") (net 6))
 (via (at 153 77) (size 0.6) (drill 0.3) (layers "F.Cu" "B.Cu") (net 6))
 (segment (start 103.61 114.39) (end 103.61 119.46) (width 0.2) (layer "B.Cu") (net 6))
 (segment (start 153 92) (end 137 108) (width 0.2) (layer "B.Cu") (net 6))
 (segment (start 153 77) (end 153 92) (width 0.2) (layer "B.Cu") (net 6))
 (segment (start 135 113.5) (end 104.5 113.5) (width 0.2) (layer "B.Cu") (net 6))
 (segment (start 104.5 113.5) (end 103.61 114.39) (width 0.2) (layer "B.Cu") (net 6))
 (segment (start 137 111.5) (end 135 113.5) (width 0.2) (layer "B.Cu") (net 6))
 (segment (start 137 108) (end 137 111.5) (width 0.2) (layer "B.Cu") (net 6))
 (segment (start 162.9492 59.8808) (end 155 59.8808) (width 0.2) (layer "F.Cu") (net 23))
 (via (at 155 59.8808) (size 0.6) (drill 0.3) (layers "F.Cu" "B.Cu") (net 23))
 (segment (start 136.5 16) (end 125 16) (width 0.2) (layer "B.Cu") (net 23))
 (segment (start 153.8808 59.8808) (end 139 45) (width 0.2) (layer "B.Cu") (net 23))
 (segment (start 139 18.5) (end 136.5 16) (width 0.2) (layer "B.Cu") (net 23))
 (segment (start 125 16) (end 123.11 17.89) (width 0.2) (layer "B.Cu") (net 23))
 (segment (start 139 45) (end 139 18.5) (width 0.2) (layer "B.Cu") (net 23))
 (segment (start 155 59.8808) (end 153.8808 59.8808) (width 0.2) (layer "B.Cu") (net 23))
 (segment (start 123.11 17.89) (end 123.11 21.96) (width 0.2) (layer "B.Cu") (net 23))
 (segment (start 138.5 38) (end 138.5 45) (width 0.2) (layer "F.Cu") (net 22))
 (segment (start 138.5 45) (end 150.8408 57.3408) (width 0.2) (layer "F.Cu") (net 22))
 (segment (start 150.8408 57.3408) (end 162.9492 57.3408) (width 0.2) (layer "F.Cu") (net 22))
 (segment (start 137.25 36.75) (end 138.5 38) (width 0.2) (layer "F.Cu") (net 22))
 (via (at 137.25 36.75) (size 0.6) (drill 0.3) (layers "F.Cu" "B.Cu") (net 22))
 (segment (start 125 35.5) (end 123.11 37.39) (width 0.2) (layer "B.Cu") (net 22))
 (segment (start 137.25 36.75) (end 136 35.5) (width 0.2) (layer "B.Cu") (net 22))
 (segment (start 136 35.5) (end 125 35.5) (width 0.2) (layer "B.Cu") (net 22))
 (segment (start 123.11 37.39) (end 123.11 41.46) (width 0.2) (layer "B.Cu") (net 22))
 (segment (start 139.434314 72) (end 139.834314 71.6) (width 0.2) (layer "B.Cu") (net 4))
 (segment (start 155.248529 70.4) (end 158.848529 74) (width 0.2) (layer "B.Cu") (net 4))
 (segment (start 153.551471 71.6) (end 154.751471 70.4) (width 0.2) (layer "B.Cu") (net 4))
 (segment (start 158.848529 74) (end 177.0684 74) (width 0.2) (layer "B.Cu") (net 4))
 (segment (start 123.11 60.96) (end 123.11 71.11) (width 0.2) (layer "B.Cu") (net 4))
 (segment (start 177.0684 74) (end 178.1892 75.1208) (width 0.2) (layer "B.Cu") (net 4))
 (segment (start 123.11 71.11) (end 124 72) (width 0.2) (layer "B.Cu") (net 4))
 (segment (start 139.834314 71.6) (end 153.551471 71.6) (width 0.2) (layer "B.Cu") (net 4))
 (segment (start 124 72) (end 139.434314 72) (width 0.2) (layer "B.Cu") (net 4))
 (segment (start 154.751471 70.4) (end 155.248529 70.4) (width 0.2) (layer "B.Cu") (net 4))
 (segment (start 180.5 77) (end 180.5 74.8916) (width 0.2) (layer "B.Cu") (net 3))
 (segment (start 180.5 74.8916) (end 178.1892 72.5808) (width 0.2) (layer "B.Cu") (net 3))
 (segment (start 124.5 92) (end 135 92) (width 0.2) (layer "B.Cu") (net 3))
 (segment (start 123.11 90.61) (end 124.5 92) (width 0.2) (layer "B.Cu") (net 3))
 (segment (start 123.11 80.46) (end 123.11 90.61) (width 0.2) (layer "B.Cu") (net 3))
 (segment (start 137 73.5) (end 137.7 72.8) (width 0.2) (layer "B.Cu") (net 3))
 (segment (start 135 92) (end 137 90) (width 0.2) (layer "B.Cu") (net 3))
 (segment (start 161 77) (end 180.5 77) (width 0.2) (layer "B.Cu") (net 3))
 (segment (start 153.765685 72.8) (end 154.584885 71.9808) (width 0.2) (layer "B.Cu") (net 3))
 (segment (start 137 90) (end 137 73.5) (width 0.2) (layer "B.Cu") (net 3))
 (segment (start 155.9808 71.9808) (end 161 77) (width 0.2) (layer "B.Cu") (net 3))
 (segment (start 137.7 72.8) (end 153.765685 72.8) (width 0.2) (layer "B.Cu") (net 3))
 (segment (start 154.584885 71.9808) (end 155.9808 71.9808) (width 0.2) (layer "B.Cu") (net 3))
 (segment (start 176.5 77.6) (end 176.5 71.73) (width 0.2) (layer "F.Cu") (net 28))
 (segment (start 137.5 105) (end 153.5 89) (width 0.2) (layer "F.Cu") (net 28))
 (segment (start 176.5 71.73) (end 178.1892 70.0408) (width 0.2) (layer "F.Cu") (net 28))
 (segment (start 153.5 89) (end 155.4 89) (width 0.2) (layer "F.Cu") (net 28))
 (segment (start 137.5 108.9) (end 137.5 105) (width 0.2) (layer "F.Cu") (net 28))
 (segment (start 136.4 110) (end 137.5 108.9) (width 0.2) (layer "F.Cu") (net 28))
 (via (at 155.4 89) (size 0.6) (drill 0.3) (layers "F.Cu" "B.Cu") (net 28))
 (via (at 136.4 110) (size 0.6) (drill 0.3) (layers "F.Cu" "B.Cu") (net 28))
 (via (at 176.5 77.6) (size 0.6) (drill 0.3) (layers "F.Cu" "B.Cu") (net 28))
 (segment (start 161 77.5) (end 176.4 77.5) (width 0.2) (layer "B.Cu") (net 28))
 (segment (start 135 111.5) (end 136.4 110.1) (width 0.2) (layer "B.Cu") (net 28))
 (segment (start 123.11 99.96) (end 123.11 110.11) (width 0.2) (layer "B.Cu") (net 28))
 (segment (start 124.5 111.5) (end 135 111.5) (width 0.2) (layer "B.Cu") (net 28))
 (segment (start 156.5 89) (end 157 88.5) (width 0.2) (layer "B.Cu") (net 28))
 (segment (start 136.4 110.1) (end 136.4 110) (width 0.2) (layer "B.Cu") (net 28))
 (segment (start 155.4 89) (end 156.5 89) (width 0.2) (layer "B.Cu") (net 28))
 (segment (start 176.4 77.5) (end 176.5 77.6) (width 0.2) (layer "B.Cu") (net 28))
 (segment (start 157 81.5) (end 161 77.5) (width 0.2) (layer "B.Cu") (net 28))
 (segment (start 157 88.5) (end 157 81.5) (width 0.2) (layer "B.Cu") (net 28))
 (segment (start 123.11 110.11) (end 124.5 111.5) (width 0.2) (layer "B.Cu") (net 28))
 (segment (start 118.5 38) (end 123 33.5) (width 0.2) (layer "F.Cu") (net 2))
 (segment (start 118.5 116.5) (end 118.5 38) (width 0.2) (layer "F.Cu") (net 2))
 (segment (start 137.5 33.5) (end 160 56) (width 0.2) (layer "F.Cu") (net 2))
 (segment (start 123 33.5) (end 128.5 33.5) (width 0.2) (layer "F.Cu") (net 2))
 (segment (start 160 56) (end 160.5 56) (width 0.2) (layer "F.Cu") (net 2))
 (via (at 128.5 33.5) (size 0.6) (drill 0.3) (layers "F.Cu" "B.Cu") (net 2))
 (via (at 160.5 56) (size 0.6) (drill 0.3) (layers "F.Cu" "B.Cu") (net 2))
 (via (at 137.5 33.5) (size 0.6) (drill 0.3) (layers "F.Cu" "B.Cu") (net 2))
 (via (at 118.5 116.5) (size 0.6) (drill 0.3) (layers "F.Cu" "B.Cu") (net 2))
 (segment (start 128.5 33.5) (end 137.5 33.5) (width 0.2) (layer "B.Cu") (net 2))
 (segment (start 160.5 56) (end 170.784035 56) (width 0.2) (layer "B.Cu") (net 2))
 (segment (start 177.0892 66.4008) (end 178.1892 67.5008) (width 0.2) (layer "B.Cu") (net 2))
 (segment (start 170.784035 56) (end 177.0892 62.305165) (width 0.2) (layer "B.Cu") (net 2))
 (segment (start 177.0892 62.305165) (end 177.0892 66.4008) (width 0.2) (layer "B.Cu") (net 2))
 (segment (start 121.46 119.46) (end 118.5 116.5) (width 0.2) (layer "B.Cu") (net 2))
 (segment (start 123.11 119.46) (end 121.46 119.46) (width 0.2) (layer "B.Cu") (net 2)))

